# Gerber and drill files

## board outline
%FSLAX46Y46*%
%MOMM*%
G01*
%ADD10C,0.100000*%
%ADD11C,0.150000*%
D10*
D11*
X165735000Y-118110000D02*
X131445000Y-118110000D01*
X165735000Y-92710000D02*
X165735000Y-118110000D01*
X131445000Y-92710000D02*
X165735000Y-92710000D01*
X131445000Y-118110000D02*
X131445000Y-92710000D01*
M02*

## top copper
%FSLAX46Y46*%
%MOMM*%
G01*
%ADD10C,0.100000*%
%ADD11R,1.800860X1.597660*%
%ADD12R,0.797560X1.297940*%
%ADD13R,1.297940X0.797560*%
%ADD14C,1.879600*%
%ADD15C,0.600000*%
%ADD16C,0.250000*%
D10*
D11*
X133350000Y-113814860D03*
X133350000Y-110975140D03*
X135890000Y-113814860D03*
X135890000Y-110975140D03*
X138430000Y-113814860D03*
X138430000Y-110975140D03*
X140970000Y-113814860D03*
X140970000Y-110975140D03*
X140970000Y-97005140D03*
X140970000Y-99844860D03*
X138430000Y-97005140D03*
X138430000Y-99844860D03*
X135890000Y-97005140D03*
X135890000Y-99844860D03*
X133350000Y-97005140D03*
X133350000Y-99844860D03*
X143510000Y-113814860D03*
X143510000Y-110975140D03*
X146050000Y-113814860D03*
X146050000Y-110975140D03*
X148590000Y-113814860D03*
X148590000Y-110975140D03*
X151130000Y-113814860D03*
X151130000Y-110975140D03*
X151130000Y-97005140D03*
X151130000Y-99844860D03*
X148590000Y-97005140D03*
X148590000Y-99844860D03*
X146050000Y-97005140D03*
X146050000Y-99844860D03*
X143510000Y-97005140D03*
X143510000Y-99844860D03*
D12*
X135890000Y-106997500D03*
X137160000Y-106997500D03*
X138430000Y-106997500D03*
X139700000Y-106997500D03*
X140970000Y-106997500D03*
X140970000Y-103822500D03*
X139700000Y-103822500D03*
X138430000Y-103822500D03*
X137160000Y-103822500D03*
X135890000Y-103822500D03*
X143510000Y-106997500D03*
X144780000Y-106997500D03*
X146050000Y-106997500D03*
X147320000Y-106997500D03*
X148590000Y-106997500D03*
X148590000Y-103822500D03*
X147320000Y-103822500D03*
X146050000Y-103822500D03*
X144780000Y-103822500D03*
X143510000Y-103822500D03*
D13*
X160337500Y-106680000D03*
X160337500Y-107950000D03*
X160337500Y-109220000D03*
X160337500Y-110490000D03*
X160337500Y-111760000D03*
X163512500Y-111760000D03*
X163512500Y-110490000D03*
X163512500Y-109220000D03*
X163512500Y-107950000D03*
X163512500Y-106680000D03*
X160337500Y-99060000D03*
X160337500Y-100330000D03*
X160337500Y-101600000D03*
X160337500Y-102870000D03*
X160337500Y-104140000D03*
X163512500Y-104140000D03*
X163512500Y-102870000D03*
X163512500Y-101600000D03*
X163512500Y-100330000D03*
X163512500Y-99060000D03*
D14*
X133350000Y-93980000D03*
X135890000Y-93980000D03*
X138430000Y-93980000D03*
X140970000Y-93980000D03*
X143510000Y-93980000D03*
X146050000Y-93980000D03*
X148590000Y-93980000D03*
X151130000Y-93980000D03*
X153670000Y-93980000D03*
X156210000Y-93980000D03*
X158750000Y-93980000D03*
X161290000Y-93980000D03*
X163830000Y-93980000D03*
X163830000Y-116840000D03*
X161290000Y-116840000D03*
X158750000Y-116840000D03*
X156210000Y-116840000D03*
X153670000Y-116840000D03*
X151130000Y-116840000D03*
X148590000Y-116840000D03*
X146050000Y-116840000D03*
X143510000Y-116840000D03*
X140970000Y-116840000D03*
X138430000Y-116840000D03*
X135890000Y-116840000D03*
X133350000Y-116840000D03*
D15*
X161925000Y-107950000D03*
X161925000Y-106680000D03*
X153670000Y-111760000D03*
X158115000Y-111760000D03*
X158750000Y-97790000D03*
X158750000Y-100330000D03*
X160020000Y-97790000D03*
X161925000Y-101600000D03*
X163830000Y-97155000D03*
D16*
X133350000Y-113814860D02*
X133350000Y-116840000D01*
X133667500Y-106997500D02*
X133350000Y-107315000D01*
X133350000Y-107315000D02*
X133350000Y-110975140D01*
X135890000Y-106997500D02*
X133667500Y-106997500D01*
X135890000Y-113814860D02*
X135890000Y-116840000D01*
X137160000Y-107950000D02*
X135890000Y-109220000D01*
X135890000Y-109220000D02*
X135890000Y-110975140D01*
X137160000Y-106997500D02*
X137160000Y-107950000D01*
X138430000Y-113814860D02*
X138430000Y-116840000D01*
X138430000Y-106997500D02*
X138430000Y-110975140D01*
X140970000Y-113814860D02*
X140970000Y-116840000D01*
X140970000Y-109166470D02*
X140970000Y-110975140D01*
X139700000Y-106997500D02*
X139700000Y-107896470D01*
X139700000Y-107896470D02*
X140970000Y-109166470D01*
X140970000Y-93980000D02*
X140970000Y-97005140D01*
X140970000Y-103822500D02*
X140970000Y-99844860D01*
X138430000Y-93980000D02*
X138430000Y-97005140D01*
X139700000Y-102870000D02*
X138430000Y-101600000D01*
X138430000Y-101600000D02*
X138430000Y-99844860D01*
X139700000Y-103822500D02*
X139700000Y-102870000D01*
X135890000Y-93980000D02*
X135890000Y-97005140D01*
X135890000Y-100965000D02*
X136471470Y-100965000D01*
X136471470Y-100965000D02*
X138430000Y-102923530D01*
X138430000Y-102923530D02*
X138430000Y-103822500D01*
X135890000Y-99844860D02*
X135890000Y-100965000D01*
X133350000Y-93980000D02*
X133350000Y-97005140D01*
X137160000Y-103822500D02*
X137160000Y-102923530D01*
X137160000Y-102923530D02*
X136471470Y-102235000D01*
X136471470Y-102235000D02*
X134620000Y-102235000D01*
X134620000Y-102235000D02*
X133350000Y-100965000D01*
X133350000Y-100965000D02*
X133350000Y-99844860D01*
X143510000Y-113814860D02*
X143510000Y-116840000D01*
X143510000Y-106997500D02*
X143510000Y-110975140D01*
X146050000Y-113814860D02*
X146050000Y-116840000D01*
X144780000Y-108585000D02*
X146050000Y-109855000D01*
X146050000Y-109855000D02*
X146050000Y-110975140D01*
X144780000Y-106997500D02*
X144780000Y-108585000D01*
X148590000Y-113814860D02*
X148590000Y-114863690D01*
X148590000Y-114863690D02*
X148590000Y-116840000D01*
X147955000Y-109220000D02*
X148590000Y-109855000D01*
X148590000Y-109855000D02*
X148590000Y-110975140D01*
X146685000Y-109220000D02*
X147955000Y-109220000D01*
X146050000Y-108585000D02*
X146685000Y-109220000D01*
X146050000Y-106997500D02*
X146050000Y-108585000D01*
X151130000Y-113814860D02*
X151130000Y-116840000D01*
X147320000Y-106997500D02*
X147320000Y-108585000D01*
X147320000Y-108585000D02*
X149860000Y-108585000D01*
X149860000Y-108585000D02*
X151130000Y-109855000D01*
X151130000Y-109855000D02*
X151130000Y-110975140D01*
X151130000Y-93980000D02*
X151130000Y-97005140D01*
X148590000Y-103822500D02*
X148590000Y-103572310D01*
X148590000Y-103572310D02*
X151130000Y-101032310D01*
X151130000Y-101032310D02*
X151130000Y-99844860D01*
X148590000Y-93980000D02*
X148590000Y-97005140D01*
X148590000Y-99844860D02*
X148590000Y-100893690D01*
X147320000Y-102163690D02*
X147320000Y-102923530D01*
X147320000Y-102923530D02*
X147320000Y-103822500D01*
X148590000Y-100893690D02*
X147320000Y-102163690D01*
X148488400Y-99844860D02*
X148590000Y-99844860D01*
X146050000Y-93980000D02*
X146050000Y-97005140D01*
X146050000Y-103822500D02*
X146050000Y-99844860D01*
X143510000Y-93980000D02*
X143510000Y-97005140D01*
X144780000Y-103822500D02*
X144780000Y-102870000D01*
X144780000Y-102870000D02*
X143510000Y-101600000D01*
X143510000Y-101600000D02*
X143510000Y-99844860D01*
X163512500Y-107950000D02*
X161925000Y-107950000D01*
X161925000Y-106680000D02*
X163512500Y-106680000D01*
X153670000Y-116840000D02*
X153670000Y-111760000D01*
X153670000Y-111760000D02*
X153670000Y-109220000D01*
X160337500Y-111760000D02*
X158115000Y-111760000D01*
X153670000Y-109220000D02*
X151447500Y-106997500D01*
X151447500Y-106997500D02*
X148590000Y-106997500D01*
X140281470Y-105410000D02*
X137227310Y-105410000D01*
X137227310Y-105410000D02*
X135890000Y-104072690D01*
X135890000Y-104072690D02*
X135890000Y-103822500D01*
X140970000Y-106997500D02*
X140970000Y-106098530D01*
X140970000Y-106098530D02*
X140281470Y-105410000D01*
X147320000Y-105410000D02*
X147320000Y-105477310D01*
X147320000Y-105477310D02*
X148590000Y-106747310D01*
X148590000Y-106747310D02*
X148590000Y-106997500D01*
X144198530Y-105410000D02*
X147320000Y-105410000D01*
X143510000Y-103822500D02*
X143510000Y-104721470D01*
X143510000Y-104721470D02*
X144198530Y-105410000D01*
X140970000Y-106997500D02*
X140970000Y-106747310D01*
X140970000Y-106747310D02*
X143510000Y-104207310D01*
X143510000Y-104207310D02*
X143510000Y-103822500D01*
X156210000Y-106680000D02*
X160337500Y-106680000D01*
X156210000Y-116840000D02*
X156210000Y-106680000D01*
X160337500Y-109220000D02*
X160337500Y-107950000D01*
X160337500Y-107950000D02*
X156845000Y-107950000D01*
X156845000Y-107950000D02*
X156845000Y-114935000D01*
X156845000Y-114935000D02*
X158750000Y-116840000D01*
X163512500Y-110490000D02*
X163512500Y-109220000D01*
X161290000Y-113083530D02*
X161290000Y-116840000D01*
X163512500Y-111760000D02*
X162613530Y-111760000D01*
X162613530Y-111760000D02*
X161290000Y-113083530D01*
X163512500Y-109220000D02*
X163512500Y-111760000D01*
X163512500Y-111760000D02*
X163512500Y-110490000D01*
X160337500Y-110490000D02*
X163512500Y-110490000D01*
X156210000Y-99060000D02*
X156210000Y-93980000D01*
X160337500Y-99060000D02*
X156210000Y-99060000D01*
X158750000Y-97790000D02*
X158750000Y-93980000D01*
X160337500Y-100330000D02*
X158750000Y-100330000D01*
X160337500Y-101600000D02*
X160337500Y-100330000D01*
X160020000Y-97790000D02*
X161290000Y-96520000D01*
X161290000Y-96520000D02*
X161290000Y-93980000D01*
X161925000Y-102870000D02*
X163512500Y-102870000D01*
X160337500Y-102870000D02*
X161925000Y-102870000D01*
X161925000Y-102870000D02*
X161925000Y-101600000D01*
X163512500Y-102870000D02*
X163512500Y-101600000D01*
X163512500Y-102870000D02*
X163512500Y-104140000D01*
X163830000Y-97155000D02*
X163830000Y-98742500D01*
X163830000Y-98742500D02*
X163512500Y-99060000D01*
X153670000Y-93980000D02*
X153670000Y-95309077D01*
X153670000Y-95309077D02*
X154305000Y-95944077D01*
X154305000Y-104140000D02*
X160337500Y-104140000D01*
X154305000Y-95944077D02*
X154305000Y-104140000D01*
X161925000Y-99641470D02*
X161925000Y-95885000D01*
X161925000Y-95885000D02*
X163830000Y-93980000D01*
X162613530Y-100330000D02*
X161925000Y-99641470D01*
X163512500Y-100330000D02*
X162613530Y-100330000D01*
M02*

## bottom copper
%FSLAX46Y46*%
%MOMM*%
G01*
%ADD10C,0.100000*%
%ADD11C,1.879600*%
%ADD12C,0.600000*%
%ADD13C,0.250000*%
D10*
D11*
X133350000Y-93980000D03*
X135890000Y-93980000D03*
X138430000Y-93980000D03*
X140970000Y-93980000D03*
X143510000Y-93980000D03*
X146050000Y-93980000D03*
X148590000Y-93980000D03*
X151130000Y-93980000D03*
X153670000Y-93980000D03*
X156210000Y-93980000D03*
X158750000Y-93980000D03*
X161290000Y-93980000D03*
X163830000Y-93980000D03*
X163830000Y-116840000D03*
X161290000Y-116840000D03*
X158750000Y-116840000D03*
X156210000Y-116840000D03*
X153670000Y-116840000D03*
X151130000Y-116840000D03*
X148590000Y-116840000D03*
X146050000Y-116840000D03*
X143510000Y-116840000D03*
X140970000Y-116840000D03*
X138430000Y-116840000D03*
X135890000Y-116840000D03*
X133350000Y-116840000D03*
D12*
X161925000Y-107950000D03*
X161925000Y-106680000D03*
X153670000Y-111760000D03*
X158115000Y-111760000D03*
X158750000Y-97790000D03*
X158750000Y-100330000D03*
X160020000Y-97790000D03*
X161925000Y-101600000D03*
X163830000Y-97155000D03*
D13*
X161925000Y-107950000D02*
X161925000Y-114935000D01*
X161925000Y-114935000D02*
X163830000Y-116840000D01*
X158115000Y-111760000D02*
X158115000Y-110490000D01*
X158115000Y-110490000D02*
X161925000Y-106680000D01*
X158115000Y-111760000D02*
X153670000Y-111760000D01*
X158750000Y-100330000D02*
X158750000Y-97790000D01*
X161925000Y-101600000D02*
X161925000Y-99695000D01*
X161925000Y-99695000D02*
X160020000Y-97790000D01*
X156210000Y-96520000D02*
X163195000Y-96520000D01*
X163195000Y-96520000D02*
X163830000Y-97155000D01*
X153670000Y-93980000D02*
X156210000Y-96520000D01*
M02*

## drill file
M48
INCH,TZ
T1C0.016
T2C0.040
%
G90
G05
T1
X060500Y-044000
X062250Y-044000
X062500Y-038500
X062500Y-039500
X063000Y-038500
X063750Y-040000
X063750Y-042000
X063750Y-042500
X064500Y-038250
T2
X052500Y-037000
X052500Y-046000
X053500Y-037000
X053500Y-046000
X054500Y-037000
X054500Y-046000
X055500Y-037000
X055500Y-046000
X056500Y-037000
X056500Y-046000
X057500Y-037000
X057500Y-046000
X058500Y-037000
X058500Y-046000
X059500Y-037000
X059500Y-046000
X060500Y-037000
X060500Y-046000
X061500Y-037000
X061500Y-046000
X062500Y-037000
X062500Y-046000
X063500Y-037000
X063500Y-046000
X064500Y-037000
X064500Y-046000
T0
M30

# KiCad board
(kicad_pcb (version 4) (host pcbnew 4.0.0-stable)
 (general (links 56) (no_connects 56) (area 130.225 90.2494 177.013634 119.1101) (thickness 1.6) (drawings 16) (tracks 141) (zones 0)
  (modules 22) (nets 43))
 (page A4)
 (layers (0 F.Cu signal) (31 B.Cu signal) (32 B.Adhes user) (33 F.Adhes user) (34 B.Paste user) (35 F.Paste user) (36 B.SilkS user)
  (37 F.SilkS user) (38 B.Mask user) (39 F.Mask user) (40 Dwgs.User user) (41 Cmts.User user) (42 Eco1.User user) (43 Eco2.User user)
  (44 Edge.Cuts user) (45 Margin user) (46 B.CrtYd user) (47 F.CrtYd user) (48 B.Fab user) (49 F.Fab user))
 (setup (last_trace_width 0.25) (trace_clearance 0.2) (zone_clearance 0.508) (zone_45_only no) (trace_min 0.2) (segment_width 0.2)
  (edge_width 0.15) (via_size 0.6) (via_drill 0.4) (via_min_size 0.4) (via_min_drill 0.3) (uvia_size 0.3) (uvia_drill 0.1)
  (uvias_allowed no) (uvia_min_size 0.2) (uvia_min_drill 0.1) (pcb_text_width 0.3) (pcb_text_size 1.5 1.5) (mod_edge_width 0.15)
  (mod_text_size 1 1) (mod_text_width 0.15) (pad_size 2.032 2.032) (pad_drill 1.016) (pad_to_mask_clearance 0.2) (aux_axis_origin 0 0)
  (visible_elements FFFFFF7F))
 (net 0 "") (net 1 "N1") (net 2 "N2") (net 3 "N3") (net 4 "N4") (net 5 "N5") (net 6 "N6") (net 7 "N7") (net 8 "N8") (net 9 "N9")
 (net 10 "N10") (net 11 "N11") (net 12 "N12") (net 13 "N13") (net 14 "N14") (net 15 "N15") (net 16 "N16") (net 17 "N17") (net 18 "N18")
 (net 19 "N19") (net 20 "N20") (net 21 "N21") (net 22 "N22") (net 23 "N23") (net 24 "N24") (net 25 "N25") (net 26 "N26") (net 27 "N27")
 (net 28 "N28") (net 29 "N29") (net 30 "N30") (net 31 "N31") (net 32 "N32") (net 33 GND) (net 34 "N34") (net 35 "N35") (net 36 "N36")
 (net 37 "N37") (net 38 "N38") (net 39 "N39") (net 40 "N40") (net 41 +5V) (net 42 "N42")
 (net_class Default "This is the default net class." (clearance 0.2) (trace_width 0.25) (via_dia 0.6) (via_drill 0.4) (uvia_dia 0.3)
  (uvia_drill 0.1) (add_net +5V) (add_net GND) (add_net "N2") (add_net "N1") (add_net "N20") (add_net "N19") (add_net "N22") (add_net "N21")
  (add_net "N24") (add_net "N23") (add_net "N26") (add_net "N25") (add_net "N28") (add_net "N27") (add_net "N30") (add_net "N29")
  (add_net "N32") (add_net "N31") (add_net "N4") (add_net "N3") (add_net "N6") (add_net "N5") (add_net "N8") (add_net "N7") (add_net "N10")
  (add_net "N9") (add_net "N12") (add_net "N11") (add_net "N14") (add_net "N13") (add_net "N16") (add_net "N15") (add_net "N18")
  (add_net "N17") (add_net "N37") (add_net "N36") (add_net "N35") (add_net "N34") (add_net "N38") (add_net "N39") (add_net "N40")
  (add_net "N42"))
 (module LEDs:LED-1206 (layer F.Cu) (at 133.35 112.395 270)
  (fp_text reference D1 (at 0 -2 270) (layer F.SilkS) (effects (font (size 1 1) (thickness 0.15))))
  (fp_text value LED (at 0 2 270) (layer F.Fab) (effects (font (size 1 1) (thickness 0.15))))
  (pad 2 smd rect (at 1.41986 0 90) (size 1.59766 1.80086) (layers F.Cu F.Paste F.Mask) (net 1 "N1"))
  (pad 1 smd rect (at -1.41986 0 90) (size 1.59766 1.80086) (layers F.Cu F.Paste F.Mask) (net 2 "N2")))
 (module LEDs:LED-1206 (layer F.Cu) (at 135.89 112.395 270)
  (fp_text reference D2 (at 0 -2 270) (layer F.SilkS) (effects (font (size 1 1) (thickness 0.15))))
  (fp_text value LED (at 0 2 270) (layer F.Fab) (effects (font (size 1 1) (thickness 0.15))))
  (pad 2 smd rect (at 1.41986 0 90) (size 1.59766 1.80086) (layers F.Cu F.Paste F.Mask) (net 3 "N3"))
  (pad 1 smd rect (at -1.41986 0 90) (size 1.59766 1.80086) (layers F.Cu F.Paste F.Mask) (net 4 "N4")))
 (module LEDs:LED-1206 (layer F.Cu) (at 138.43 112.395 270)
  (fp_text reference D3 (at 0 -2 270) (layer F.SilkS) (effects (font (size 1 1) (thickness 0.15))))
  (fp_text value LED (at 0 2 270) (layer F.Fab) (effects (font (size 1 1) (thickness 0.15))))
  (pad 2 smd rect (at 1.41986 0 90) (size 1.59766 1.80086) (layers F.Cu F.Paste F.Mask) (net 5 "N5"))
  (pad 1 smd rect (at -1.41986 0 90) (size 1.59766 1.80086) (layers F.Cu F.Paste F.Mask) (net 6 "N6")))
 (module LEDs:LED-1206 (layer F.Cu) (at 140.97 112.395 270)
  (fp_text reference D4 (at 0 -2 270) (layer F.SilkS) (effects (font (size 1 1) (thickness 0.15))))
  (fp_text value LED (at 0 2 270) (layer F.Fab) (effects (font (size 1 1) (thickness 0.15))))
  (pad 2 smd rect (at 1.41986 0 90) (size 1.59766 1.80086) (layers F.Cu F.Paste F.Mask) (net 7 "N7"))
  (pad 1 smd rect (at -1.41986 0 90) (size 1.59766 1.80086) (layers F.Cu F.Paste F.Mask) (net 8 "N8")))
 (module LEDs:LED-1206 (layer F.Cu) (at 140.97 98.425 90)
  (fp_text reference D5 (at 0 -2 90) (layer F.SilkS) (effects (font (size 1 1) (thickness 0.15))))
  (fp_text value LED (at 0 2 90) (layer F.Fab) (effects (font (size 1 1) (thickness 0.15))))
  (pad 2 smd rect (at 1.41986 0 270) (size 1.59766 1.80086) (layers F.Cu F.Paste F.Mask) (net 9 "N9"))
  (pad 1 smd rect (at -1.41986 0 270) (size 1.59766 1.80086) (layers F.Cu F.Paste F.Mask) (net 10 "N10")))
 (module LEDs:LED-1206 (layer F.Cu) (at 138.43 98.425 90)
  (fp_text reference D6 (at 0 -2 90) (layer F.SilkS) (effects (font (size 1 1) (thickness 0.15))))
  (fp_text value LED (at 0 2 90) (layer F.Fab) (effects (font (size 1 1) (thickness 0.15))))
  (pad 2 smd rect (at 1.41986 0 270) (size 1.59766 1.80086) (layers F.Cu F.Paste F.Mask) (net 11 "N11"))
  (pad 1 smd rect (at -1.41986 0 270) (size 1.59766 1.80086) (layers F.Cu F.Paste F.Mask) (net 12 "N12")))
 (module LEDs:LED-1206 (layer F.Cu) (at 135.89 98.425 90)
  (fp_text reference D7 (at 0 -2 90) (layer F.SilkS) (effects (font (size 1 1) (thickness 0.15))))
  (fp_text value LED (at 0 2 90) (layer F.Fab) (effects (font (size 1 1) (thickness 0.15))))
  (pad 2 smd rect (at 1.41986 0 270) (size 1.59766 1.80086) (layers F.Cu F.Paste F.Mask) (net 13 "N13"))
  (pad 1 smd rect (at -1.41986 0 270) (size 1.59766 1.80086) (layers F.Cu F.Paste F.Mask) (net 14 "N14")))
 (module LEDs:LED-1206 (layer F.Cu) (at 133.35 98.425 90)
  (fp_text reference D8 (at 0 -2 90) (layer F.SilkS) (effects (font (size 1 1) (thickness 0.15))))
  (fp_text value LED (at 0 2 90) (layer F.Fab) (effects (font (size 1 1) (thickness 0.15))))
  (pad 2 smd rect (at 1.41986 0 270) (size 1.59766 1.80086) (layers F.Cu F.Paste F.Mask) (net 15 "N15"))
  (pad 1 smd rect (at -1.41986 0 270) (size 1.59766 1.80086) (layers F.Cu F.Paste F.Mask) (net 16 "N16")))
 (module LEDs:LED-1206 (layer F.Cu) (at 143.51 112.395 270)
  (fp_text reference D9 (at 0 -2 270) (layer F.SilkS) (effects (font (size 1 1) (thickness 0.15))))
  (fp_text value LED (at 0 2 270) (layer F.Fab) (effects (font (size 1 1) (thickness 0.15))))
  (pad 2 smd rect (at 1.41986 0 90) (size 1.59766 1.80086) (layers F.Cu F.Paste F.Mask) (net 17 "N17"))
  (pad 1 smd rect (at -1.41986 0 90) (size 1.59766 1.80086) (layers F.Cu F.Paste F.Mask) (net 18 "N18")))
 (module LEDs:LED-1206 (layer F.Cu) (at 146.05 112.395 270)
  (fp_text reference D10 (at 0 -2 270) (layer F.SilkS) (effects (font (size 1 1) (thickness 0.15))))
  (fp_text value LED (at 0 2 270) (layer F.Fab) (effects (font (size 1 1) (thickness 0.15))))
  (pad 2 smd rect (at 1.41986 0 90) (size 1.59766 1.80086) (layers F.Cu F.Paste F.Mask) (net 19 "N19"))
  (pad 1 smd rect (at -1.41986 0 90) (size 1.59766 1.80086) (layers F.Cu F.Paste F.Mask) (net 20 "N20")))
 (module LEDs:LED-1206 (layer F.Cu) (at 148.59 112.395 270)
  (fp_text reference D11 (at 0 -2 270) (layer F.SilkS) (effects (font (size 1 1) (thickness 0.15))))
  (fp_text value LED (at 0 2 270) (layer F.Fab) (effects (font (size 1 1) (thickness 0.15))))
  (pad 2 smd rect (at 1.41986 0 90) (size 1.59766 1.80086) (layers F.Cu F.Paste F.Mask) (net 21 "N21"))
  (pad 1 smd rect (at -1.41986 0 90) (size 1.59766 1.80086) (layers F.Cu F.Paste F.Mask) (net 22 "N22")))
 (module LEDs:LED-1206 (layer F.Cu) (at 151.13 112.395 270)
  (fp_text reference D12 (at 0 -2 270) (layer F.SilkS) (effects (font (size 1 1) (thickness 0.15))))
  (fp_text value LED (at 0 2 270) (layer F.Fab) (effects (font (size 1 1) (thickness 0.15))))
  (pad 2 smd rect (at 1.41986 0 90) (size 1.59766 1.80086) (layers F.Cu F.Paste F.Mask) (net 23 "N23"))
  (pad 1 smd rect (at -1.41986 0 90) (size 1.59766 1.80086) (layers F.Cu F.Paste F.Mask) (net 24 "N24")))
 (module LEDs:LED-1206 (layer F.Cu) (at 151.13 98.425 90)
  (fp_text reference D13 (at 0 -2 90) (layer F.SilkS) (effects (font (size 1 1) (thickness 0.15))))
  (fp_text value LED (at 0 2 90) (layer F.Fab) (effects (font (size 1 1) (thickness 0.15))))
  (pad 2 smd rect (at 1.41986 0 270) (size 1.59766 1.80086) (layers F.Cu F.Paste F.Mask) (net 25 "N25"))
  (pad 1 smd rect (at -1.41986 0 270) (size 1.59766 1.80086) (layers F.Cu F.Paste F.Mask) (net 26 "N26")))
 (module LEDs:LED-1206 (layer F.Cu) (at 148.59 98.425 90)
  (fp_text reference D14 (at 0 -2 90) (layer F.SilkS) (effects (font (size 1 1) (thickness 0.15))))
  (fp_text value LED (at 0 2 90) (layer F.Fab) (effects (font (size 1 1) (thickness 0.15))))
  (pad 2 smd rect (at 1.41986 0 270) (size 1.59766 1.80086) (layers F.Cu F.Paste F.Mask) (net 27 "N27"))
  (pad 1 smd rect (at -1.41986 0 270) (size 1.59766 1.80086) (layers F.Cu F.Paste F.Mask) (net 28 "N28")))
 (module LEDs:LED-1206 (layer F.Cu) (at 146.05 98.425 90)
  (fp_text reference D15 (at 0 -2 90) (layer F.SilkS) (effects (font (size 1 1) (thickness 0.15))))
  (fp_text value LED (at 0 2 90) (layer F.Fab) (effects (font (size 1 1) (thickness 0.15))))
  (pad 2 smd rect (at 1.41986 0 270) (size 1.59766 1.80086) (layers F.Cu F.Paste F.Mask) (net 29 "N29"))
  (pad 1 smd rect (at -1.41986 0 270) (size 1.59766 1.80086) (layers F.Cu F.Paste F.Mask) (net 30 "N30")))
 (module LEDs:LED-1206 (layer F.Cu) (at 143.51 98.425 90)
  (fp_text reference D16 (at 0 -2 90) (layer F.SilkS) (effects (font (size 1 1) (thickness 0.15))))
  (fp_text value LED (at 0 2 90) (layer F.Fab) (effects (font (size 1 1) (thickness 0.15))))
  (pad 2 smd rect (at 1.41986 0 270) (size 1.59766 1.80086) (layers F.Cu F.Paste F.Mask) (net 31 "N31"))
  (pad 1 smd rect (at -1.41986 0 270) (size 1.59766 1.80086) (layers F.Cu F.Paste F.Mask) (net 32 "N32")))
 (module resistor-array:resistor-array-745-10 (layer F.Cu) (at 138.43 105.41)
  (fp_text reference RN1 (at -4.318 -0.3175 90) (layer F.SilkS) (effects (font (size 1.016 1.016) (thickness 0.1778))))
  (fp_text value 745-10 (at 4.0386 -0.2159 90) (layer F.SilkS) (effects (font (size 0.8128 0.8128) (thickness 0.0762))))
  (pad 1 smd rect (at -2.54 1.5875) (size 0.79756 1.29794) (layers F.Cu F.Paste F.Mask) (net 2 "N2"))
  (pad 2 smd rect (at -1.27 1.5875) (size 0.79756 1.29794) (layers F.Cu F.Paste F.Mask) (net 4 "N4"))
  (pad 3 smd rect (at 0 1.5875) (size 0.79756 1.29794) (layers F.Cu F.Paste F.Mask) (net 6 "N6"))
  (pad 4 smd rect (at 1.27 1.5875) (size 0.79756 1.29794) (layers F.Cu F.Paste F.Mask) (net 8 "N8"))
  (pad 5 smd rect (at 2.54 1.5875) (size 0.79756 1.29794) (layers F.Cu F.Paste F.Mask) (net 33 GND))
  (pad 6 smd rect (at 2.54 -1.5875) (size 0.79756 1.29794) (layers F.Cu F.Paste F.Mask) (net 10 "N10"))
  (pad 7 smd rect (at 1.27 -1.5875) (size 0.79756 1.29794) (layers F.Cu F.Paste F.Mask) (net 12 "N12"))
  (pad 8 smd rect (at 0 -1.5875) (size 0.79756 1.29794) (layers F.Cu F.Paste F.Mask) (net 14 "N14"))
  (pad 9 smd rect (at -1.27 -1.5875) (size 0.79756 1.29794) (layers F.Cu F.Paste F.Mask) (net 16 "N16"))
  (pad 10 smd rect (at -2.54 -1.5875) (size 0.79756 1.29794) (layers F.Cu F.Paste F.Mask) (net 33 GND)))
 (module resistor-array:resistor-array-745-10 (layer F.Cu) (at 146.05 105.41)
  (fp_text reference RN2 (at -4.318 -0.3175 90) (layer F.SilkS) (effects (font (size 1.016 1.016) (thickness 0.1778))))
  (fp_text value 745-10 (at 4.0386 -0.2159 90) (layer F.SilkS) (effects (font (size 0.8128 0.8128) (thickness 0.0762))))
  (pad 1 smd rect (at -2.54 1.5875) (size 0.79756 1.29794) (layers F.Cu F.Paste F.Mask) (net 18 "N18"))
  (pad 2 smd rect (at -1.27 1.5875) (size 0.79756 1.29794) (layers F.Cu F.Paste F.Mask) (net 20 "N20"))
  (pad 3 smd rect (at 0 1.5875) (size 0.79756 1.29794) (layers F.Cu F.Paste F.Mask) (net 22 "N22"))
  (pad 4 smd rect (at 1.27 1.5875) (size 0.79756 1.29794) (layers F.Cu F.Paste F.Mask) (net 24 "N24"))
  (pad 5 smd rect (at 2.54 1.5875) (size 0.79756 1.29794) (layers F.Cu F.Paste F.Mask) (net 33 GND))
  (pad 6 smd rect (at 2.54 -1.5875) (size 0.79756 1.29794) (layers F.Cu F.Paste F.Mask) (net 26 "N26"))
  (pad 7 smd rect (at 1.27 -1.5875) (size 0.79756 1.29794) (layers F.Cu F.Paste F.Mask) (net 28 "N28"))
  (pad 8 smd rect (at 0 -1.5875) (size 0.79756 1.29794) (layers F.Cu F.Paste F.Mask) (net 30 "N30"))
  (pad 9 smd rect (at -1.27 -1.5875) (size 0.79756 1.29794) (layers F.Cu F.Paste F.Mask) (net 32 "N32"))
  (pad 10 smd rect (at -2.54 -1.5875) (size 0.79756 1.29794) (layers F.Cu F.Paste F.Mask) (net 33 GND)))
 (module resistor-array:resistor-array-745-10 (layer F.Cu) (at 161.925 109.22 270)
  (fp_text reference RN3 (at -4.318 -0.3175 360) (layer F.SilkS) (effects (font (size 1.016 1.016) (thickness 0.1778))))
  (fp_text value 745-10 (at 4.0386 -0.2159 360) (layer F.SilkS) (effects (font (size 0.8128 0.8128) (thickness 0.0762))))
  (pad 1 smd rect (at -2.54 1.5875 270) (size 0.79756 1.29794) (layers F.Cu F.Paste F.Mask) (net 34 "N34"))
  (pad 2 smd rect (at -1.27 1.5875 270) (size 0.79756 1.29794) (layers F.Cu F.Paste F.Mask) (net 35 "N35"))
  (pad 3 smd rect (at 0 1.5875 270) (size 0.79756 1.29794) (layers F.Cu F.Paste F.Mask) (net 35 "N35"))
  (pad 4 smd rect (at 1.27 1.5875 270) (size 0.79756 1.29794) (layers F.Cu F.Paste F.Mask) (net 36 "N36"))
  (pad 5 smd rect (at 2.54 1.5875 270) (size 0.79756 1.29794) (layers F.Cu F.Paste F.Mask) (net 33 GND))
  (pad 6 smd rect (at 2.54 -1.5875 270) (size 0.79756 1.29794) (layers F.Cu F.Paste F.Mask) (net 36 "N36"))
  (pad 7 smd rect (at 1.27 -1.5875 270) (size 0.79756 1.29794) (layers F.Cu F.Paste F.Mask) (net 36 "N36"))
  (pad 8 smd rect (at 0 -1.5875 270) (size 0.79756 1.29794) (layers F.Cu F.Paste F.Mask) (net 36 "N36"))
  (pad 9 smd rect (at -1.27 -1.5875 270) (size 0.79756 1.29794) (layers F.Cu F.Paste F.Mask) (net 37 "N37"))
  (pad 10 smd rect (at -2.54 -1.5875 270) (size 0.79756 1.29794) (layers F.Cu F.Paste F.Mask) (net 33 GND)))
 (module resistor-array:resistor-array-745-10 (layer F.Cu) (at 161.925 101.6 270)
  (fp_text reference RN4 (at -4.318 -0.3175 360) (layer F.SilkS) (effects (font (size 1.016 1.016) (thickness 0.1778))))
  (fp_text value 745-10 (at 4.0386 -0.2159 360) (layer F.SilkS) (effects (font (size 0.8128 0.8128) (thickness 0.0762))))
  (pad 1 smd rect (at -2.54 1.5875 270) (size 0.79756 1.29794) (layers F.Cu F.Paste F.Mask) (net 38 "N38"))
  (pad 2 smd rect (at -1.27 1.5875 270) (size 0.79756 1.29794) (layers F.Cu F.Paste F.Mask) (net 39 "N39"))
  (pad 3 smd rect (at 0 1.5875 270) (size 0.79756 1.29794) (layers F.Cu F.Paste F.Mask) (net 39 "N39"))
  (pad 4 smd rect (at 1.27 1.5875 270) (size 0.79756 1.29794) (layers F.Cu F.Paste F.Mask) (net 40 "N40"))
  (pad 5 smd rect (at 2.54 1.5875 270) (size 0.79756 1.29794) (layers F.Cu F.Paste F.Mask) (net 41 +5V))
  (pad 6 smd rect (at 2.54 -1.5875 270) (size 0.79756 1.29794) (layers F.Cu F.Paste F.Mask) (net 40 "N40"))
  (pad 7 smd rect (at 1.27 -1.5875 270) (size 0.79756 1.29794) (layers F.Cu F.Paste F.Mask) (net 40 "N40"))
  (pad 8 smd rect (at 0 -1.5875 270) (size 0.79756 1.29794) (layers F.Cu F.Paste F.Mask) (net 40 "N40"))
  (pad 9 smd rect (at -1.27 -1.5875 270) (size 0.79756 1.29794) (layers F.Cu F.Paste F.Mask) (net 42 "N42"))
  (pad 10 smd rect (at -2.54 -1.5875 270) (size 0.79756 1.29794) (layers F.Cu F.Paste F.Mask) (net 41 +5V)))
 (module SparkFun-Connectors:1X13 (layer F.Cu) (at 133.35 93.98)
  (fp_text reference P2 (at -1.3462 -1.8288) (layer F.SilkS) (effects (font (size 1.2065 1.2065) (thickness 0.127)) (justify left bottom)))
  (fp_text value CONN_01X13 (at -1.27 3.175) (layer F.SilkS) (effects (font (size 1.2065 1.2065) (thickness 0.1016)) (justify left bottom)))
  (pad 1 thru_hole circle (at 0 0 90) (size 1.8796 1.8796) (drill 1.016) (layers *.Cu *.Mask) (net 15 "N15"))
  (pad 2 thru_hole circle (at 2.54 0 90) (size 1.8796 1.8796) (drill 1.016) (layers *.Cu *.Mask) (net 13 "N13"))
  (pad 3 thru_hole circle (at 5.08 0 90) (size 1.8796 1.8796) (drill 1.016) (layers *.Cu *.Mask) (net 11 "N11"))
  (pad 4 thru_hole circle (at 7.62 0 90) (size 1.8796 1.8796) (drill 1.016) (layers *.Cu *.Mask) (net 9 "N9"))
  (pad 5 thru_hole circle (at 10.16 0 90) (size 1.8796 1.8796) (drill 1.016) (layers *.Cu *.Mask) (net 31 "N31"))
  (pad 6 thru_hole circle (at 12.7 0 90) (size 1.8796 1.8796) (drill 1.016) (layers *.Cu *.Mask) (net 29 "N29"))
  (pad 7 thru_hole circle (at 15.24 0 90) (size 1.8796 1.8796) (drill 1.016) (layers *.Cu *.Mask) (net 27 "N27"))
  (pad 8 thru_hole circle (at 17.78 0 90) (size 1.8796 1.8796) (drill 1.016) (layers *.Cu *.Mask) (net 25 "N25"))
  (pad 9 thru_hole circle (at 20.32 0 90) (size 1.8796 1.8796) (drill 1.016) (layers *.Cu *.Mask) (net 41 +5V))
  (pad 10 thru_hole circle (at 22.86 0 90) (size 1.8796 1.8796) (drill 1.016) (layers *.Cu *.Mask) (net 38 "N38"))
  (pad 11 thru_hole circle (at 25.4 0 90) (size 1.8796 1.8796) (drill 1.016) (layers *.Cu *.Mask) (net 39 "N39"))
  (pad 12 thru_hole circle (at 27.94 0 90) (size 1.8796 1.8796) (drill 1.016) (layers *.Cu *.Mask) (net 40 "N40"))
  (pad 13 thru_hole circle (at 30.48 0 90) (size 1.8796 1.8796) (drill 1.016) (layers *.Cu *.Mask) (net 42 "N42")))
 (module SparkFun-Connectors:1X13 (layer F.Cu) (at 163.83 116.84 180)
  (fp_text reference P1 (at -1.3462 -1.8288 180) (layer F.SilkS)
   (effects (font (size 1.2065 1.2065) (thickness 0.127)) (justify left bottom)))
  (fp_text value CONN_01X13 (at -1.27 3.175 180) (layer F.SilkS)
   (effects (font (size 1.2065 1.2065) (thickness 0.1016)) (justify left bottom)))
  (pad 1 thru_hole circle (at 0 0 270) (size 1.8796 1.8796) (drill 1.016) (layers *.Cu *.Mask) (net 37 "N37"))
  (pad 2 thru_hole circle (at 2.54 0 270) (size 1.8796 1.8796) (drill 1.016) (layers *.Cu *.Mask) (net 36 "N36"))
  (pad 3 thru_hole circle (at 5.08 0 270) (size 1.8796 1.8796) (drill 1.016) (layers *.Cu *.Mask) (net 35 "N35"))
  (pad 4 thru_hole circle (at 7.62 0 270) (size 1.8796 1.8796) (drill 1.016) (layers *.Cu *.Mask) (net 34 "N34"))
  (pad 5 thru_hole circle (at 10.16 0 270) (size 1.8796 1.8796) (drill 1.016) (layers *.Cu *.Mask) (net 33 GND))
  (pad 6 thru_hole circle (at 12.7 0 270) (size 1.8796 1.8796) (drill 1.016) (layers *.Cu *.Mask) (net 23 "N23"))
  (pad 7 thru_hole circle (at 15.24 0 270) (size 1.8796 1.8796) (drill 1.016) (layers *.Cu *.Mask) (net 21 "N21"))
  (pad 8 thru_hole circle (at 17.78 0 270) (size 1.8796 1.8796) (drill 1.016) (layers *.Cu *.Mask) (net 19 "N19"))
  (pad 9 thru_hole circle (at 20.32 0 270) (size 1.8796 1.8796) (drill 1.016) (layers *.Cu *.Mask) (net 17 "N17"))
  (pad 10 thru_hole circle (at 22.86 0 270) (size 1.8796 1.8796) (drill 1.016) (layers *.Cu *.Mask) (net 7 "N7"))
  (pad 11 thru_hole circle (at 25.4 0 270) (size 1.8796 1.8796) (drill 1.016) (layers *.Cu *.Mask) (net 5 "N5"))
  (pad 12 thru_hole circle (at 27.94 0 270) (size 1.8796 1.8796) (drill 1.016) (layers *.Cu *.Mask) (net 3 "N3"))
  (pad 13 thru_hole circle (at 30.48 0 270) (size 1.8796 1.8796) (drill 1.016) (layers *.Cu *.Mask) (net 1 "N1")))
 (gr_line (start 165.735 118.11) (end 131.445 118.11) (layer Edge.Cuts) (width 0.15))
 (gr_line (start 165.735 92.71) (end 165.735 118.11) (layer Edge.Cuts) (width 0.15))
 (gr_line (start 131.445 92.71) (end 165.735 92.71) (layer Edge.Cuts) (width 0.15))
 (gr_line (start 131.445 118.11) (end 131.445 92.71) (layer Edge.Cuts) (width 0.15))
 (segment (start 133.35 113.81486) (end 133.35 116.84) (width 0.25) (layer F.Cu) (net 1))
 (segment (start 133.6675 106.9975) (end 133.35 107.315) (width 0.25) (layer F.Cu) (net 2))
 (segment (start 133.35 107.315) (end 133.35 110.97514) (width 0.25) (layer F.Cu) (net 2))
 (segment (start 135.89 106.9975) (end 133.6675 106.9975) (width 0.25) (layer F.Cu) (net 2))
 (segment (start 135.89 113.81486) (end 135.89 116.84) (width 0.25) (layer F.Cu) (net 3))
 (segment (start 137.16 107.95) (end 135.89 109.22) (width 0.25) (layer F.Cu) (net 4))
 (segment (start 135.89 109.22) (end 135.89 110.97514) (width 0.25) (layer F.Cu) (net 4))
 (segment (start 137.16 106.9975) (end 137.16 107.95) (width 0.25) (layer F.Cu) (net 4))
 (segment (start 138.43 113.81486) (end 138.43 116.84) (width 0.25) (layer F.Cu) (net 5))
 (segment (start 138.43 106.9975) (end 138.43 110.97514) (width 0.25) (layer F.Cu) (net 6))
 (segment (start 140.97 113.81486) (end 140.97 116.84) (width 0.25) (layer F.Cu) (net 7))
 (segment (start 140.97 109.16647) (end 140.97 110.97514) (width 0.25) (layer F.Cu) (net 8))
 (segment (start 139.7 106.9975) (end 139.7 107.89647) (width 0.25) (layer F.Cu) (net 8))
 (segment (start 139.7 107.89647) (end 140.97 109.16647) (width 0.25) (layer F.Cu) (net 8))
 (segment (start 140.97 93.98) (end 140.97 97.00514) (width 0.25) (layer F.Cu) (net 9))
 (segment (start 140.97 103.8225) (end 140.97 99.84486) (width 0.25) (layer F.Cu) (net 10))
 (segment (start 138.43 93.98) (end 138.43 97.00514) (width 0.25) (layer F.Cu) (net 11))
 (segment (start 139.7 102.87) (end 138.43 101.6) (width 0.25) (layer F.Cu) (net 12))
 (segment (start 138.43 101.6) (end 138.43 99.84486) (width 0.25) (layer F.Cu) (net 12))
 (segment (start 139.7 103.8225) (end 139.7 102.87) (width 0.25) (layer F.Cu) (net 12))
 (segment (start 135.89 93.98) (end 135.89 97.00514) (width 0.25) (layer F.Cu) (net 13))
 (segment (start 135.89 100.965) (end 136.47147 100.965) (width 0.25) (layer F.Cu) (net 14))
 (segment (start 136.47147 100.965) (end 138.43 102.92353) (width 0.25) (layer F.Cu) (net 14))
 (segment (start 138.43 102.92353) (end 138.43 103.8225) (width 0.25) (layer F.Cu) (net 14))
 (segment (start 135.89 99.84486) (end 135.89 100.965) (width 0.25) (layer F.Cu) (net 14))
 (segment (start 133.35 93.98) (end 133.35 97.00514) (width 0.25) (layer F.Cu) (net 15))
 (segment (start 137.16 103.8225) (end 137.16 102.92353) (width 0.25) (layer F.Cu) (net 16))
 (segment (start 137.16 102.92353) (end 136.47147 102.235) (width 0.25) (layer F.Cu) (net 16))
 (segment (start 136.47147 102.235) (end 134.62 102.235) (width 0.25) (layer F.Cu) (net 16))
 (segment (start 134.62 102.235) (end 133.35 100.965) (width 0.25) (layer F.Cu) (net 16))
 (segment (start 133.35 100.965) (end 133.35 99.84486) (width 0.25) (layer F.Cu) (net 16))
 (segment (start 143.51 113.81486) (end 143.51 116.84) (width 0.25) (layer F.Cu) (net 17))
 (segment (start 143.51 106.9975) (end 143.51 110.97514) (width 0.25) (layer F.Cu) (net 18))
 (segment (start 146.05 113.81486) (end 146.05 116.84) (width 0.25) (layer F.Cu) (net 19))
 (segment (start 144.78 108.585) (end 146.05 109.855) (width 0.25) (layer F.Cu) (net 20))
 (segment (start 146.05 109.855) (end 146.05 110.97514) (width 0.25) (layer F.Cu) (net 20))
 (segment (start 144.78 106.9975) (end 144.78 108.585) (width 0.25) (layer F.Cu) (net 20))
 (segment (start 148.59 113.81486) (end 148.59 114.86369) (width 0.25) (layer F.Cu) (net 21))
 (segment (start 148.59 114.86369) (end 148.59 116.84) (width 0.25) (layer F.Cu) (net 21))
 (segment (start 147.955 109.22) (end 148.59 109.855) (width 0.25) (layer F.Cu) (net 22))
 (segment (start 148.59 109.855) (end 148.59 110.97514) (width 0.25) (layer F.Cu) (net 22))
 (segment (start 146.685 109.22) (end 147.955 109.22) (width 0.25) (layer F.Cu) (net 22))
 (segment (start 146.05 108.585) (end 146.685 109.22) (width 0.25) (layer F.Cu) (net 22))
 (segment (start 146.05 106.9975) (end 146.05 108.585) (width 0.25) (layer F.Cu) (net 22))
 (segment (start 151.13 113.81486) (end 151.13 116.84) (width 0.25) (layer F.Cu) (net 23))
 (segment (start 147.32 106.9975) (end 147.32 108.585) (width 0.25) (layer F.Cu) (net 24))
 (segment (start 147.32 108.585) (end 149.86 108.585) (width 0.25) (layer F.Cu) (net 24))
 (segment (start 149.86 108.585) (end 151.13 109.855) (width 0.25) (layer F.Cu) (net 24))
 (segment (start 151.13 109.855) (end 151.13 110.97514) (width 0.25) (layer F.Cu) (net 24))
 (segment (start 151.13 93.98) (end 151.13 97.00514) (width 0.25) (layer F.Cu) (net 25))
 (segment (start 148.59 103.8225) (end 148.59 103.57231) (width 0.25) (layer F.Cu) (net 26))
 (segment (start 148.59 103.57231) (end 151.13 101.03231) (width 0.25) (layer F.Cu) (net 26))
 (segment (start 151.13 101.03231) (end 151.13 99.84486) (width 0.25) (layer F.Cu) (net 26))
 (segment (start 148.59 93.98) (end 148.59 97.00514) (width 0.25) (layer F.Cu) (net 27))
 (segment (start 148.59 99.84486) (end 148.59 100.89369) (width 0.25) (layer F.Cu) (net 28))
 (segment (start 147.32 102.16369) (end 147.32 102.92353) (width 0.25) (layer F.Cu) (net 28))
 (segment (start 147.32 102.92353) (end 147.32 103.8225) (width 0.25) (layer F.Cu) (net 28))
 (segment (start 148.59 100.89369) (end 147.32 102.16369) (width 0.25) (layer F.Cu) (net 28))
 (segment (start 148.4884 99.84486) (end 148.59 99.84486) (width 0.25) (layer F.Cu) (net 28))
 (segment (start 146.05 93.98) (end 146.05 97.00514) (width 0.25) (layer F.Cu) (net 29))
 (segment (start 146.05 103.8225) (end 146.05 99.84486) (width 0.25) (layer F.Cu) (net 30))
 (segment (start 143.51 93.98) (end 143.51 97.00514) (width 0.25) (layer F.Cu) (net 31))
 (segment (start 144.78 103.8225) (end 144.78 102.87) (width 0.25) (layer F.Cu) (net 32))
 (segment (start 144.78 102.87) (end 143.51 101.6) (width 0.25) (layer F.Cu) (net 32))
 (segment (start 143.51 101.6) (end 143.51 99.84486) (width 0.25) (layer F.Cu) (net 32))
 (segment (start 161.925 107.95) (end 161.925 114.935) (width 0.25) (layer B.Cu) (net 37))
 (segment (start 161.925 114.935) (end 163.83 116.84) (width 0.25) (layer B.Cu) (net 37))
 (segment (start 163.5125 107.95) (end 161.925 107.95) (width 0.25) (layer F.Cu) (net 37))
 (via (at 161.925 107.95) (size 0.6) (drill 0.4) (layers F.Cu B.Cu) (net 37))
 (segment (start 161.925 106.68) (end 163.5125 106.68) (width 0.25) (layer F.Cu) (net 33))
 (segment (start 158.115 111.76) (end 158.115 110.49) (width 0.25) (layer B.Cu) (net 33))
 (segment (start 158.115 110.49) (end 161.925 106.68) (width 0.25) (layer B.Cu) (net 33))
 (via (at 161.925 106.68) (size 0.6) (drill 0.4) (layers F.Cu B.Cu) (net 33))
 (segment (start 153.67 116.84) (end 153.67 111.76) (width 0.25) (layer F.Cu) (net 33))
 (segment (start 153.67 111.76) (end 153.67 109.22) (width 0.25) (layer F.Cu) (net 33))
 (segment (start 158.115 111.76) (end 153.67 111.76) (width 0.25) (layer B.Cu) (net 33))
 (via (at 153.67 111.76) (size 0.6) (drill 0.4) (layers F.Cu B.Cu) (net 33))
 (segment (start 160.3375 111.76) (end 158.115 111.76) (width 0.25) (layer F.Cu) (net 33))
 (via (at 158.115 111.76) (size 0.6) (drill 0.4) (layers F.Cu B.Cu) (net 33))
 (segment (start 153.67 109.22) (end 151.4475 106.9975) (width 0.25) (layer F.Cu) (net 33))
 (segment (start 151.4475 106.9975) (end 148.59 106.9975) (width 0.25) (layer F.Cu) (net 33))
 (segment (start 140.28147 105.41) (end 137.22731 105.41) (width 0.25) (layer F.Cu) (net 33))
 (segment (start 137.22731 105.41) (end 135.89 104.07269) (width 0.25) (layer F.Cu) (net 33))
 (segment (start 135.89 104.07269) (end 135.89 103.8225) (width 0.25) (layer F.Cu) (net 33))
 (segment (start 140.97 106.9975) (end 140.97 106.09853) (width 0.25) (layer F.Cu) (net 33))
 (segment (start 140.97 106.09853) (end 140.28147 105.41) (width 0.25) (layer F.Cu) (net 33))
 (segment (start 147.32 105.41) (end 147.32 105.47731) (width 0.25) (layer F.Cu) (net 33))
 (segment (start 147.32 105.47731) (end 148.59 106.74731) (width 0.25) (layer F.Cu) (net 33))
 (segment (start 148.59 106.74731) (end 148.59 106.9975) (width 0.25) (layer F.Cu) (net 33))
 (segment (start 144.19853 105.41) (end 147.32 105.41) (width 0.25) (layer F.Cu) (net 33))
 (segment (start 143.51 103.8225) (end 143.51 104.72147) (width 0.25) (layer F.Cu) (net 33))
 (segment (start 143.51 104.72147) (end 144.19853 105.41) (width 0.25) (layer F.Cu) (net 33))
 (segment (start 140.97 106.9975) (end 140.97 106.74731) (width 0.25) (layer F.Cu) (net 33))
 (segment (start 140.97 106.74731) (end 143.51 104.20731) (width 0.25) (layer F.Cu) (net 33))
 (segment (start 143.51 104.20731) (end 143.51 103.8225) (width 0.25) (layer F.Cu) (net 33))
 (segment (start 156.21 106.68) (end 160.3375 106.68) (width 0.25) (layer F.Cu) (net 34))
 (segment (start 156.21 116.84) (end 156.21 106.68) (width 0.25) (layer F.Cu) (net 34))
 (segment (start 160.3375 109.22) (end 160.3375 107.95) (width 0.25) (layer F.Cu) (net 35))
 (segment (start 160.3375 107.95) (end 156.845 107.95) (width 0.25) (layer F.Cu) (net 35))
 (segment (start 156.845 107.95) (end 156.845 114.935) (width 0.25) (layer F.Cu) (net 35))
 (segment (start 156.845 114.935) (end 158.75 116.84) (width 0.25) (layer F.Cu) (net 35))
 (segment (start 163.5125 110.49) (end 163.5125 109.22) (width 0.25) (layer F.Cu) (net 36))
 (segment (start 161.29 113.08353) (end 161.29 116.84) (width 0.25) (layer F.Cu) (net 36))
 (segment (start 163.5125 111.76) (end 162.61353 111.76) (width 0.25) (layer F.Cu) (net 36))
 (segment (start 162.61353 111.76) (end 161.29 113.08353) (width 0.25) (layer F.Cu) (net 36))
 (segment (start 163.5125 109.22) (end 163.5125 111.76) (width 0.25) (layer F.Cu) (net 36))
 (segment (start 163.5125 111.76) (end 163.5125 110.49) (width 0.25) (layer F.Cu) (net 36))
 (segment (start 160.3375 110.49) (end 163.5125 110.49) (width 0.25) (layer F.Cu) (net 36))
 (segment (start 156.21 99.06) (end 156.21 93.98) (width 0.25) (layer F.Cu) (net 38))
 (segment (start 160.3375 99.06) (end 156.21 99.06) (width 0.25) (layer F.Cu) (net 38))
 (segment (start 158.75 97.79) (end 158.75 93.98) (width 0.25) (layer F.Cu) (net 39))
 (segment (start 158.75 100.33) (end 158.75 97.79) (width 0.25) (layer B.Cu) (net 39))
 (via (at 158.75 97.79) (size 0.6) (drill 0.4) (layers F.Cu B.Cu) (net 39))
 (via (at 158.75 100.33) (size 0.6) (drill 0.4) (layers F.Cu B.Cu) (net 39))
 (segment (start 160.3375 100.33) (end 158.75 100.33) (width 0.25) (layer F.Cu) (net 39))
 (segment (start 160.3375 101.6) (end 160.3375 100.33) (width 0.25) (layer F.Cu) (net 39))
 (segment (start 160.02 97.79) (end 161.29 96.52) (width 0.25) (layer F.Cu) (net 40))
 (segment (start 161.29 96.52) (end 161.29 93.98) (width 0.25) (layer F.Cu) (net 40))
 (segment (start 161.925 101.6) (end 161.925 99.695) (width 0.25) (layer B.Cu) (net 40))
 (segment (start 161.925 99.695) (end 160.02 97.79) (width 0.25) (layer B.Cu) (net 40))
 (via (at 160.02 97.79) (size 0.6) (drill 0.4) (layers F.Cu B.Cu) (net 40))
 (segment (start 161.925 102.87) (end 163.5125 102.87) (width 0.25) (layer F.Cu) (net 40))
 (via (at 161.925 101.6) (size 0.6) (drill 0.4) (layers F.Cu B.Cu) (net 40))
 (segment (start 160.3375 102.87) (end 161.925 102.87) (width 0.25) (layer F.Cu) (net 40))
 (segment (start 161.925 102.87) (end 161.925 101.6) (width 0.25) (layer F.Cu) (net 40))
 (segment (start 163.5125 102.87) (end 163.5125 101.6) (width 0.25) (layer F.Cu) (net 40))
 (segment (start 163.5125 102.87) (end 163.5125 104.14) (width 0.25) (layer F.Cu) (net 40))
 (segment (start 163.83 97.155) (end 163.83 98.7425) (width 0.25) (layer F.Cu) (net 41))
 (segment (start 163.83 98.7425) (end 163.5125 99.06) (width 0.25) (layer F.Cu) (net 41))
 (segment (start 156.21 96.52) (end 163.195 96.52) (width 0.25) (layer B.Cu) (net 41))
 (segment (start 163.195 96.52) (end 163.83 97.155) (width 0.25) (layer B.Cu) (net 41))
 (via (at 163.83 97.155) (size 0.6) (drill 0.4) (layers F.Cu B.Cu) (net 41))
 (segment (start 153.67 93.98) (end 156.21 96.52) (width 0.25) (layer B.Cu) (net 41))
 (segment (start 153.67 93.98) (end 153.67 95.309077) (width 0.25) (layer F.Cu) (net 41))
 (segment (start 153.67 95.309077) (end 154.305 95.944077) (width 0.25) (layer F.Cu) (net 41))
 (segment (start 154.305 104.14) (end 160.3375 104.14) (width 0.25) (layer F.Cu) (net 41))
 (segment (start 154.305 95.944077) (end 154.305 104.14) (width 0.25) (layer F.Cu) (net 41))
 (segment (start 161.925 99.64147) (end 161.925 95.885) (width 0.25) (layer F.Cu) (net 42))
 (segment (start 161.925 95.885) (end 163.83 93.98) (width 0.25) (layer F.Cu) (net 42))
 (segment (start 162.61353 100.33) (end 161.925 99.64147) (width 0.25) (layer F.Cu) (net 42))
 (segment (start 163.5125 100.33) (end 162.61353 100.33) (width 0.25) (layer F.Cu) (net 42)))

